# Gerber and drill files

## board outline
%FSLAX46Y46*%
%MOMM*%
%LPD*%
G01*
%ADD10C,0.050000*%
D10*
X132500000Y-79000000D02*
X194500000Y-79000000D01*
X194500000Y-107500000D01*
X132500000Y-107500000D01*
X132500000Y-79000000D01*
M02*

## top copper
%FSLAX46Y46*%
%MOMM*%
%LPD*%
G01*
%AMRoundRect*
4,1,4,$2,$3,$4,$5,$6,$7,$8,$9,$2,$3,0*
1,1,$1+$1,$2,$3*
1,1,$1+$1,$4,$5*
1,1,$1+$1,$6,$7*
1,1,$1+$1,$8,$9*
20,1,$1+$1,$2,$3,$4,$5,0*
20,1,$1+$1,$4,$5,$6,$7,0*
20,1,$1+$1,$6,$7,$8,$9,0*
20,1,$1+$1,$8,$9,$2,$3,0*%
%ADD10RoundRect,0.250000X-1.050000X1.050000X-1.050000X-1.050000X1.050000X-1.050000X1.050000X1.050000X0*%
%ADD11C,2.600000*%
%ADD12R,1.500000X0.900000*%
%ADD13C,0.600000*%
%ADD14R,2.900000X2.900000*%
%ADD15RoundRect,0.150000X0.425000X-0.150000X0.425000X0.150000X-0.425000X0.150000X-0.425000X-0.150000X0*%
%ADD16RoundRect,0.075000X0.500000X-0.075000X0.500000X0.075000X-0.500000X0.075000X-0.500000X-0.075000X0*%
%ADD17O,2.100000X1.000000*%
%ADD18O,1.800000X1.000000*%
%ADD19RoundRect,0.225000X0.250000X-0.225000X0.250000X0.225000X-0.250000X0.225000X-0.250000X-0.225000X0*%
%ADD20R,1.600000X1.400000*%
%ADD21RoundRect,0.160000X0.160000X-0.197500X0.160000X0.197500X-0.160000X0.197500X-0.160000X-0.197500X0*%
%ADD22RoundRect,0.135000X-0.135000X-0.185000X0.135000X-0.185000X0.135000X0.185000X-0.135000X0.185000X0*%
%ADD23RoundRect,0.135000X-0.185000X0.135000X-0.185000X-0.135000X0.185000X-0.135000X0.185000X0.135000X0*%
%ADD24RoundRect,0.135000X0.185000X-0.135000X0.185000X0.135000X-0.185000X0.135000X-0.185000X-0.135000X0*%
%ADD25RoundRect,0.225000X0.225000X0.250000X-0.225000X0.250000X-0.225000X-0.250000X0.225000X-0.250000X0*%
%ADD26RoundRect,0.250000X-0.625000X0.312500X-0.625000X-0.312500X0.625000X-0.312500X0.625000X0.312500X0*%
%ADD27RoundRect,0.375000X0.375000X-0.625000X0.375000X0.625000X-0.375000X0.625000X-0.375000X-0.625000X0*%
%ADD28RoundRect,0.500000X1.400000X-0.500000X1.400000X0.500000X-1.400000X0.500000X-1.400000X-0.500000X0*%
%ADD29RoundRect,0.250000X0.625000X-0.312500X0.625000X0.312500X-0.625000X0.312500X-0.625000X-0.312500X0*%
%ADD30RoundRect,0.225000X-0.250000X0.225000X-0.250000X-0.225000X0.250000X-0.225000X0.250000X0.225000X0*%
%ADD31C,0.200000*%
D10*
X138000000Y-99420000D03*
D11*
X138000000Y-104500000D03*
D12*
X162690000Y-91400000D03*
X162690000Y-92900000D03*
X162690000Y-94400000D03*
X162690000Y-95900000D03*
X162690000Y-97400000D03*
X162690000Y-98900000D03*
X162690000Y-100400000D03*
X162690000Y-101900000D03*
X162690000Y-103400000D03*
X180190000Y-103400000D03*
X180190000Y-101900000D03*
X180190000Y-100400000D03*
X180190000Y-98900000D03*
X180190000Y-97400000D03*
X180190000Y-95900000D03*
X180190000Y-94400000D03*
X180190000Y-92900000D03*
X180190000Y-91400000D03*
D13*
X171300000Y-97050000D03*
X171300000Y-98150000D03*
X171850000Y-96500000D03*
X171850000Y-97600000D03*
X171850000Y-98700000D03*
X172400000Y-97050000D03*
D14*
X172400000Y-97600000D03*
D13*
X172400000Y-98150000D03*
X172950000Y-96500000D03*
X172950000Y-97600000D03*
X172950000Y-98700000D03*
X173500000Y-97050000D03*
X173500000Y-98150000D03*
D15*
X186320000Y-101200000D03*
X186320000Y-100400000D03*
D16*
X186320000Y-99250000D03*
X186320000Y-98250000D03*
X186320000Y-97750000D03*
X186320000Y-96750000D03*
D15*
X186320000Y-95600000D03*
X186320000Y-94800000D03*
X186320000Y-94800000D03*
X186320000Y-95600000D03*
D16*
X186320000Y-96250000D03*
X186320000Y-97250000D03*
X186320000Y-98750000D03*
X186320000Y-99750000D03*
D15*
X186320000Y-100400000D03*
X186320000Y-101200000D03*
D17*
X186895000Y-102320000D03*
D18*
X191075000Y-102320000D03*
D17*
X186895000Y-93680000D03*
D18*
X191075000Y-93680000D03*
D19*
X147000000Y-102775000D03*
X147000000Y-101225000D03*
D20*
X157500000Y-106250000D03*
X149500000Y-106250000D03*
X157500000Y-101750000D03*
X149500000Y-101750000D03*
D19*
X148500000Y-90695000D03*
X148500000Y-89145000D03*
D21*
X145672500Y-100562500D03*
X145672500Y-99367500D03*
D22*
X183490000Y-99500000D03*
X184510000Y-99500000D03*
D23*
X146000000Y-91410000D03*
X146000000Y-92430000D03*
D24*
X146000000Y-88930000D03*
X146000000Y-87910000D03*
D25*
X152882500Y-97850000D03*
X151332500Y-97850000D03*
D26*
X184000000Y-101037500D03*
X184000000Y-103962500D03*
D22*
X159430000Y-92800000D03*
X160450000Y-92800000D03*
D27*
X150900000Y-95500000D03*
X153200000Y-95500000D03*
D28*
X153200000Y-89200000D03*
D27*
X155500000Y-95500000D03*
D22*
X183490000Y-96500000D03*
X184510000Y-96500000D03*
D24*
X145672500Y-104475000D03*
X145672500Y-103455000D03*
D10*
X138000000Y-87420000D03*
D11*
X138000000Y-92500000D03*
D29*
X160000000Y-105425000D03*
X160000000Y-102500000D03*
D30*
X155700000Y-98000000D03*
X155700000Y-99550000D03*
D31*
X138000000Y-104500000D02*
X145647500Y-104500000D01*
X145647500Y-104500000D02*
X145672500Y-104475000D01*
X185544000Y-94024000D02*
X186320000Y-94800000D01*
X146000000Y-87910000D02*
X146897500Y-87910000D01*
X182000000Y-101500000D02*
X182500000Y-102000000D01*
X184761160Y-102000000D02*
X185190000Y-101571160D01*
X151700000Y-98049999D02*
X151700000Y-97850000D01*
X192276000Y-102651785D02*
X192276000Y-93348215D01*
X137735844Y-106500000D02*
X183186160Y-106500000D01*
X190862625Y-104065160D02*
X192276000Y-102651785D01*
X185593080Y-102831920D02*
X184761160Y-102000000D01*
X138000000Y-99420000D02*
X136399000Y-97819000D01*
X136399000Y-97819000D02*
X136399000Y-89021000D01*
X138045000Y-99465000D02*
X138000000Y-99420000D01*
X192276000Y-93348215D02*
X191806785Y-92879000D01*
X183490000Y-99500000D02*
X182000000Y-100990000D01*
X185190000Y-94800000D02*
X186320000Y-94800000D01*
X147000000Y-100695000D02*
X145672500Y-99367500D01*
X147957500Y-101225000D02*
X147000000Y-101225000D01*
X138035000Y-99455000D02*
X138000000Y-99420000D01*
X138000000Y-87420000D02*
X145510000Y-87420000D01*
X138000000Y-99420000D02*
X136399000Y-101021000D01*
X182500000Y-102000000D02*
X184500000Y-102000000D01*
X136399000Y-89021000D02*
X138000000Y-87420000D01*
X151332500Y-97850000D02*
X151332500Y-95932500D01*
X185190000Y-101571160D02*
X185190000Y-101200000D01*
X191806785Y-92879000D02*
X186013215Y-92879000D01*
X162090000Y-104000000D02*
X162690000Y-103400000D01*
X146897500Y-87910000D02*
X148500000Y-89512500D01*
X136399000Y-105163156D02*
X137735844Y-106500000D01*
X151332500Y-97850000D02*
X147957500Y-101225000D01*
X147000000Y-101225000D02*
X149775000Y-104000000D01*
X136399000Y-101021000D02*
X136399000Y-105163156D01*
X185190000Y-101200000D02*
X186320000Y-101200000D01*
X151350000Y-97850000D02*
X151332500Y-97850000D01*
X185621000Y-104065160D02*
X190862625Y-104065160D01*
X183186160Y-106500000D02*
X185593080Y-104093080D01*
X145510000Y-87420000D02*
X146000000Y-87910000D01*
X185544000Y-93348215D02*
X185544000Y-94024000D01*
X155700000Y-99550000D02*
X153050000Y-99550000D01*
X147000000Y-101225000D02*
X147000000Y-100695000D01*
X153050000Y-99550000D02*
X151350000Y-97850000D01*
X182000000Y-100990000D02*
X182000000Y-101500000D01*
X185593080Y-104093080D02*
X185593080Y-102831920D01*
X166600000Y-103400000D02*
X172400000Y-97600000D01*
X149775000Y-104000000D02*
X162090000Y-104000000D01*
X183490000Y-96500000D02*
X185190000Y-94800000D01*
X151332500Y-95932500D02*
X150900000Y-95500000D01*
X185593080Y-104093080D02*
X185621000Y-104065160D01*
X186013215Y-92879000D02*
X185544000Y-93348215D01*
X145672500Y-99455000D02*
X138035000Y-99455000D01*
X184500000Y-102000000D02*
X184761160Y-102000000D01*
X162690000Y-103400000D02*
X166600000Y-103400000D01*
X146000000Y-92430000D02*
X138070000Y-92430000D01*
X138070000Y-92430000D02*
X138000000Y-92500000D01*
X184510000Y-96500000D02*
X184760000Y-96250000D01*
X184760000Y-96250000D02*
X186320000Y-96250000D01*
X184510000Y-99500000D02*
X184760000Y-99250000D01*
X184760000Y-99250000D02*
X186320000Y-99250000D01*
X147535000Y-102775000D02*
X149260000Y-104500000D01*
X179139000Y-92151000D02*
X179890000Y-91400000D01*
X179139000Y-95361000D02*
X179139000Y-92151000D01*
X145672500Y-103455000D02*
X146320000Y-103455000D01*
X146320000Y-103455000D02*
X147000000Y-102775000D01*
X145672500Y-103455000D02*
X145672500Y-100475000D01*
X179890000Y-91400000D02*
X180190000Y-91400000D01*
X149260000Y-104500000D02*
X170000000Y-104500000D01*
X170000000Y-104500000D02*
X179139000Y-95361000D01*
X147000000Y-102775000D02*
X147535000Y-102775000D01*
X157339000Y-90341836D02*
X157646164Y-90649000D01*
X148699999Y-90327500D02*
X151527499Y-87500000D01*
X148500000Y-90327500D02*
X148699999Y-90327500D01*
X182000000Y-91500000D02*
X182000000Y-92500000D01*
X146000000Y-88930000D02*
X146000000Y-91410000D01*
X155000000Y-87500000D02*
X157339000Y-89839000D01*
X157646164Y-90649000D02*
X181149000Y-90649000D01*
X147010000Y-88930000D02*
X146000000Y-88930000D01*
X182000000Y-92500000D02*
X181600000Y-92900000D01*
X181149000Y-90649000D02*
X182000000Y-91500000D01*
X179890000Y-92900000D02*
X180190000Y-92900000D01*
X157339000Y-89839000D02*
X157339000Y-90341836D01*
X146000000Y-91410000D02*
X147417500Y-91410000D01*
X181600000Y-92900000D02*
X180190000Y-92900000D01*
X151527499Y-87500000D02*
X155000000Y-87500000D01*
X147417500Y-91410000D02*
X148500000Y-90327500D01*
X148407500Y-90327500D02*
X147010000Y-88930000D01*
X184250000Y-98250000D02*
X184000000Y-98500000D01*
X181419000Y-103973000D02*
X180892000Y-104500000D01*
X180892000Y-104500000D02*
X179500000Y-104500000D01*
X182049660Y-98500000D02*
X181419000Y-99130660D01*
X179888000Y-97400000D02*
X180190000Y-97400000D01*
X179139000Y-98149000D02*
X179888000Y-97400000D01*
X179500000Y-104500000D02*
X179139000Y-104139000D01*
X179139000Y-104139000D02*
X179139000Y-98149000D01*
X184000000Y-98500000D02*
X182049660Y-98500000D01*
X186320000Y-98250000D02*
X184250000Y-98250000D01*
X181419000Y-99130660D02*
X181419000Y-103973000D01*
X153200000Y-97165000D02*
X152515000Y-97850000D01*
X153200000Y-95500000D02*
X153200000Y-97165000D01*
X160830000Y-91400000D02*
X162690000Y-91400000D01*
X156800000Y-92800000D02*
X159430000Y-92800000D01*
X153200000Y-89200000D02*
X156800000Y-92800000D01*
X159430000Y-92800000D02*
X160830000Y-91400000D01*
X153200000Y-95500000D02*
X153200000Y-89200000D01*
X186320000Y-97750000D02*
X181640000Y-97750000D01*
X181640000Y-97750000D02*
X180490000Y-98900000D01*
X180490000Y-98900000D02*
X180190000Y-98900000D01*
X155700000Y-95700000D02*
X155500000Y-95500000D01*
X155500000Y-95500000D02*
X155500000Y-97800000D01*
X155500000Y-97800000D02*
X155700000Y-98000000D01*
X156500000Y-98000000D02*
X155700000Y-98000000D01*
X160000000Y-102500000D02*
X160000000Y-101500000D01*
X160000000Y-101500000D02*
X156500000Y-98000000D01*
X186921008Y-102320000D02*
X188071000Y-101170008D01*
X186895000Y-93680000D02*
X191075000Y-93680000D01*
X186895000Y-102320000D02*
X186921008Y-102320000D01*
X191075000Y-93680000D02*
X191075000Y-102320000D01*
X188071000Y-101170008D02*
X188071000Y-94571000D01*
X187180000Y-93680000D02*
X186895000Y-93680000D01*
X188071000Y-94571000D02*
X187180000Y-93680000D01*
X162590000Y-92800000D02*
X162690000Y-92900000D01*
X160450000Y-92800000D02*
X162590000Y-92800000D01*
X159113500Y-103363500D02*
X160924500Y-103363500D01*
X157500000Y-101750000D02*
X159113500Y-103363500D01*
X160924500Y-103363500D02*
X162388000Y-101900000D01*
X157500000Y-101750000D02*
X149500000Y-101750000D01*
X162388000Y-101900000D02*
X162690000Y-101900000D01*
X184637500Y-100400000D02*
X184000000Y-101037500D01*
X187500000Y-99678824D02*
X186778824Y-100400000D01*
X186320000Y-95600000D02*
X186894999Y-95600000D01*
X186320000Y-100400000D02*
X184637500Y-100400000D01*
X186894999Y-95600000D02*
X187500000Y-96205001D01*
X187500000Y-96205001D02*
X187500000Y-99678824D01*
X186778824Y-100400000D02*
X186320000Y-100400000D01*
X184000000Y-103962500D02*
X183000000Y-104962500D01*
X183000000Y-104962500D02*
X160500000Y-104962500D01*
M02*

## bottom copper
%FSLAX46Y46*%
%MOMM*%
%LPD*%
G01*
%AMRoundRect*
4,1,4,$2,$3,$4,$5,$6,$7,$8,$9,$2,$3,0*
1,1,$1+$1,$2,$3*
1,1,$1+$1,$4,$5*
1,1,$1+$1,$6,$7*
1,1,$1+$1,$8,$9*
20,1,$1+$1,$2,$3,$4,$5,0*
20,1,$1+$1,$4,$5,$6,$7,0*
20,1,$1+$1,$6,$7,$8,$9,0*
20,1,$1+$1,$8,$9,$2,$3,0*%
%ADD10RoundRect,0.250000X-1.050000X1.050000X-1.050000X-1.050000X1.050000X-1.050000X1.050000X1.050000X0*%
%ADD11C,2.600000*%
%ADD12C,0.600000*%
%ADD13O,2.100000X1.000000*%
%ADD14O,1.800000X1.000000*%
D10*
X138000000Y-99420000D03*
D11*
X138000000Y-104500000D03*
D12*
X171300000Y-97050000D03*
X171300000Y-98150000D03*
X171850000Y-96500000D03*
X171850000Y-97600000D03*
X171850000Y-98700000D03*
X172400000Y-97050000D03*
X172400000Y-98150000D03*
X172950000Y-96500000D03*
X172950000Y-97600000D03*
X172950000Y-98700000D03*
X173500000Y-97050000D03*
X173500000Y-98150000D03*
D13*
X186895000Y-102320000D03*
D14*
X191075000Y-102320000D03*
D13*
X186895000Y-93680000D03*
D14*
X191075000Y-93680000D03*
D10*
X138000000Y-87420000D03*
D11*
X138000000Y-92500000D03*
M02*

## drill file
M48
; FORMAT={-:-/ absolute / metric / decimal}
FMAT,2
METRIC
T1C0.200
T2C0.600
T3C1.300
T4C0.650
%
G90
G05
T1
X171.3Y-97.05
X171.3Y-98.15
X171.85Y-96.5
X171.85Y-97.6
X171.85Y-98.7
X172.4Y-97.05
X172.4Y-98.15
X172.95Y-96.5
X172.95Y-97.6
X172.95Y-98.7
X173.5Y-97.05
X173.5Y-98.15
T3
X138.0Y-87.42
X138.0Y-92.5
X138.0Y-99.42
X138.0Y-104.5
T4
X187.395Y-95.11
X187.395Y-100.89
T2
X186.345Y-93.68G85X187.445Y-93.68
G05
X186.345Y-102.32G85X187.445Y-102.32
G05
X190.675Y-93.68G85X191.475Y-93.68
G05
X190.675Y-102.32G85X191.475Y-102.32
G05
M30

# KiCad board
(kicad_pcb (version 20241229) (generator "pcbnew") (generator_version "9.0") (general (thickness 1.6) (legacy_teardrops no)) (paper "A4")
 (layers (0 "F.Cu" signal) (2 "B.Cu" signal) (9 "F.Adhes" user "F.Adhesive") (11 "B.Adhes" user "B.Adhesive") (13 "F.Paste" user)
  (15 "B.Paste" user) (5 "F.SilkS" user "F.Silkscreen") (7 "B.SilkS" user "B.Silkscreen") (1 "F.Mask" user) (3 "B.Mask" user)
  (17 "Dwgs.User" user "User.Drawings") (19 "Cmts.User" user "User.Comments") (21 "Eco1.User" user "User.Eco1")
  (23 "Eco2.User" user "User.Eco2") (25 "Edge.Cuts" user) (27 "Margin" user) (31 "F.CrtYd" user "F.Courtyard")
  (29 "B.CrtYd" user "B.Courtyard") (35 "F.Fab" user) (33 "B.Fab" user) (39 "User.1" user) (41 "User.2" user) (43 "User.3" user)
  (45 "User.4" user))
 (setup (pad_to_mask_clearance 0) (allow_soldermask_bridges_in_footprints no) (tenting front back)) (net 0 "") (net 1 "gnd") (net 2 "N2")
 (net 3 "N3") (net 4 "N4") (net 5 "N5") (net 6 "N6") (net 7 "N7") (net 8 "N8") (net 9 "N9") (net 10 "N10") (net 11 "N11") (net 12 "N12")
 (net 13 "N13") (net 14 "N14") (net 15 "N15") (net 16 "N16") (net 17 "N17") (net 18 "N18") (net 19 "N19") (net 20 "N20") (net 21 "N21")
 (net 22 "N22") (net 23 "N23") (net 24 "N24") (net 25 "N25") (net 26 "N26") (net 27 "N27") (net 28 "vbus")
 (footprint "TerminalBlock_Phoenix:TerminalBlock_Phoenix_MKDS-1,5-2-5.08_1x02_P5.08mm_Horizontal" (layer "F.Cu") (at 138 99.42 -90)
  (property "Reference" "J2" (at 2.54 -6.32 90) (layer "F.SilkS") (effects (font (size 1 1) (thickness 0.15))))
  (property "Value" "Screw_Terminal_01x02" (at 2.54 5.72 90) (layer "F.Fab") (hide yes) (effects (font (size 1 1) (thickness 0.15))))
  (pad "1" thru_hole roundrect (at 0 0 270) (size 2.6 2.6) (drill 1.3) (layers "*.Cu" "*.Mask") (remove_unused_layers no)
   (roundrect_rratio 0.096154) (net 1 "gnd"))
  (pad "2" thru_hole circle (at 5.08 0 270) (size 2.6 2.6) (drill 1.3) (layers "*.Cu" "*.Mask") (remove_unused_layers no) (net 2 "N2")))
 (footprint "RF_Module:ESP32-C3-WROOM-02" (layer "F.Cu") (at 171.44 97.4)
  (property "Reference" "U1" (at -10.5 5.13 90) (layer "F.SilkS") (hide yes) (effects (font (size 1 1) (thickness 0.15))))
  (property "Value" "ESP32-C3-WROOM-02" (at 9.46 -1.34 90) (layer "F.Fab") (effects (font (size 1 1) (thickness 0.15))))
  (pad "" smd rect (at -0.14 -0.9) (size 0.7 0.7) (layers "F.Paste"))
  (pad "" smd rect (at -0.14 0.2) (size 0.7 0.7) (layers "F.Paste"))
  (pad "" smd rect (at -0.14 1.3) (size 0.7 0.7) (layers "F.Paste"))
  (pad "" smd rect (at 0.96 -0.9) (size 0.7 0.7) (layers "F.Paste"))
  (pad "" smd rect (at 0.96 0.2) (size 0.7 0.7) (layers "F.Paste"))
  (pad "" smd rect (at 0.96 1.3) (size 0.7 0.7) (layers "F.Paste"))
  (pad "" smd rect (at 2.06 -0.9) (size 0.7 0.7) (layers "F.Paste"))
  (pad "" smd rect (at 2.06 0.2) (size 0.7 0.7) (layers "F.Paste"))
  (pad "" smd rect (at 2.06 1.3) (size 0.7 0.7) (layers "F.Paste"))
  (pad "1" smd rect (at -8.75 -6) (size 1.5 0.9) (layers "F.Cu" "F.Mask" "F.Paste") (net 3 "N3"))
  (pad "2" smd rect (at -8.75 -4.5) (size 1.5 0.9) (layers "F.Cu" "F.Mask" "F.Paste") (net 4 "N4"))
  (pad "3" smd rect (at -8.75 -3) (size 1.5 0.9) (layers "F.Cu" "F.Mask" "F.Paste") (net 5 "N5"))
  (pad "4" smd rect (at -8.75 -1.5) (size 1.5 0.9) (layers "F.Cu" "F.Mask" "F.Paste") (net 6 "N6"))
  (pad "5" smd rect (at -8.75 0) (size 1.5 0.9) (layers "F.Cu" "F.Mask" "F.Paste") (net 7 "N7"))
  (pad "6" smd rect (at -8.75 1.5) (size 1.5 0.9) (layers "F.Cu" "F.Mask" "F.Paste") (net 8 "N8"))
  (pad "7" smd rect (at -8.75 3) (size 1.5 0.9) (layers "F.Cu" "F.Mask" "F.Paste") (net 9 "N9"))
  (pad "8" smd rect (at -8.75 4.5) (size 1.5 0.9) (layers "F.Cu" "F.Mask" "F.Paste") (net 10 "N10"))
  (pad "9" smd rect (at -8.75 6) (size 1.5 0.9) (layers "F.Cu" "F.Mask" "F.Paste") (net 1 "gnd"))
  (pad "10" smd rect (at 8.75 6) (size 1.5 0.9) (layers "F.Cu" "F.Mask" "F.Paste") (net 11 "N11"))
  (pad "11" smd rect (at 8.75 4.5) (size 1.5 0.9) (layers "F.Cu" "F.Mask" "F.Paste") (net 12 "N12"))
  (pad "12" smd rect (at 8.75 3) (size 1.5 0.9) (layers "F.Cu" "F.Mask" "F.Paste") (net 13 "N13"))
  (pad "13" smd rect (at 8.75 1.5) (size 1.5 0.9) (layers "F.Cu" "F.Mask" "F.Paste") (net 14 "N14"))
  (pad "14" smd rect (at 8.75 0) (size 1.5 0.9) (layers "F.Cu" "F.Mask" "F.Paste") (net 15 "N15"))
  (pad "15" smd rect (at 8.75 -1.5) (size 1.5 0.9) (layers "F.Cu" "F.Mask" "F.Paste") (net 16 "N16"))
  (pad "16" smd rect (at 8.75 -3) (size 1.5 0.9) (layers "F.Cu" "F.Mask" "F.Paste") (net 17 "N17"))
  (pad "17" smd rect (at 8.75 -4.5) (size 1.5 0.9) (layers "F.Cu" "F.Mask" "F.Paste") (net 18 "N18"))
  (pad "18" smd rect (at 8.75 -6) (size 1.5 0.9) (layers "F.Cu" "F.Mask" "F.Paste") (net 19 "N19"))
  (pad "19" thru_hole circle (at -0.14 -0.35) (size 0.6 0.6) (drill 0.2) (layers "*.Cu" "F.Mask") (remove_unused_layers no) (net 1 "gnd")
   (zone_connect 2))
  (pad "19" thru_hole circle (at -0.14 0.75) (size 0.6 0.6) (drill 0.2) (layers "*.Cu" "F.Mask") (remove_unused_layers no) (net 1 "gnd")
   (zone_connect 2))
  (pad "19" thru_hole circle (at 0.41 -0.9) (size 0.6 0.6) (drill 0.2) (layers "*.Cu" "F.Mask") (remove_unused_layers no) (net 1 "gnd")
   (zone_connect 2))
  (pad "19" thru_hole circle (at 0.41 0.2) (size 0.6 0.6) (drill 0.2) (layers "*.Cu" "F.Mask") (remove_unused_layers no) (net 1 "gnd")
   (zone_connect 2))
  (pad "19" thru_hole circle (at 0.41 1.3) (size 0.6 0.6) (drill 0.2) (layers "*.Cu" "F.Mask") (remove_unused_layers no) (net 1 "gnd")
   (zone_connect 2))
  (pad "19" thru_hole circle (at 0.96 -0.35) (size 0.6 0.6) (drill 0.2) (layers "*.Cu" "F.Mask") (remove_unused_layers no) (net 1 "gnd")
   (zone_connect 2))
  (pad "19" smd rect (at 0.96 0.2) (size 2.9 2.9) (layers "F.Cu" "F.Mask") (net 1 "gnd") (zone_connect 2))
  (pad "19" thru_hole circle (at 0.96 0.75) (size 0.6 0.6) (drill 0.2) (layers "*.Cu" "F.Mask") (remove_unused_layers no) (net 1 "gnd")
   (zone_connect 2))
  (pad "19" thru_hole circle (at 1.51 -0.9) (size 0.6 0.6) (drill 0.2) (layers "*.Cu" "F.Mask") (remove_unused_layers no) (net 1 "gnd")
   (zone_connect 2))
  (pad "19" thru_hole circle (at 1.51 0.2) (size 0.6 0.6) (drill 0.2) (layers "*.Cu" "F.Mask") (remove_unused_layers no) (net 1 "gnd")
   (zone_connect 2))
  (pad "19" thru_hole circle (at 1.51 1.3) (size 0.6 0.6) (drill 0.2) (layers "*.Cu" "F.Mask") (remove_unused_layers no) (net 1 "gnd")
   (zone_connect 2))
  (pad "19" thru_hole circle (at 2.06 -0.35) (size 0.6 0.6) (drill 0.2) (layers "*.Cu" "F.Mask") (remove_unused_layers no) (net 1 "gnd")
   (zone_connect 2))
  (pad "19" thru_hole circle (at 2.06 0.75) (size 0.6 0.6) (drill 0.2) (layers "*.Cu" "F.Mask") (remove_unused_layers no) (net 1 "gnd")
   (zone_connect 2))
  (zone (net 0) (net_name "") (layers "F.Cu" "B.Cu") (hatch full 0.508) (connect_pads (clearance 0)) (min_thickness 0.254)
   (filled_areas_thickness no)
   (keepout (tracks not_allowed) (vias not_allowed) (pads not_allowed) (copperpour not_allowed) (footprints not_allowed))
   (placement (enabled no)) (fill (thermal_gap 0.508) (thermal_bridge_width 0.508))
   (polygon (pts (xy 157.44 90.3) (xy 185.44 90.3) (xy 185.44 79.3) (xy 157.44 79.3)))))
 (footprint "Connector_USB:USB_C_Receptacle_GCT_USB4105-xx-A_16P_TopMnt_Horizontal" (layer "F.Cu") (at 190 98 90)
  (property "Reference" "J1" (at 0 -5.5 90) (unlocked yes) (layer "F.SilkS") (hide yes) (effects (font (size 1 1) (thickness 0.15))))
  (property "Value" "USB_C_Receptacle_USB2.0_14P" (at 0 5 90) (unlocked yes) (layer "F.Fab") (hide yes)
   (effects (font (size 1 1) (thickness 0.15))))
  (pad "" np_thru_hole circle (at -2.89 -2.605 90) (size 0.65 0.65) (drill 0.65) (layers "*.Cu" "*.Mask"))
  (pad "" np_thru_hole circle (at 2.89 -2.605 90) (size 0.65 0.65) (drill 0.65) (layers "*.Cu" "*.Mask"))
  (pad "A1" smd roundrect (at -3.2 -3.68 90) (size 0.6 1.15) (layers "F.Cu" "F.Mask" "F.Paste") (roundrect_rratio 0.25) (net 1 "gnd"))
  (pad "A4" smd roundrect (at -2.4 -3.68 90) (size 0.6 1.15) (layers "F.Cu" "F.Mask" "F.Paste") (roundrect_rratio 0.25) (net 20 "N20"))
  (pad "A5" smd roundrect (at -1.25 -3.68 90) (size 0.3 1.15) (layers "F.Cu" "F.Mask" "F.Paste") (roundrect_rratio 0.25) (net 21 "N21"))
  (pad "A6" smd roundrect (at -0.25 -3.68 90) (size 0.3 1.15) (layers "F.Cu" "F.Mask" "F.Paste") (roundrect_rratio 0.25) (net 15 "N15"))
  (pad "A7" smd roundrect (at 0.25 -3.68 90) (size 0.3 1.15) (layers "F.Cu" "F.Mask" "F.Paste") (roundrect_rratio 0.25) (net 14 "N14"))
  (pad "A8" smd roundrect (at 1.25 -3.68 90) (size 0.3 1.15) (layers "F.Cu" "F.Mask" "F.Paste") (roundrect_rratio 0.25))
  (pad "A9" smd roundrect (at 2.4 -3.68 90) (size 0.6 1.15) (layers "F.Cu" "F.Mask" "F.Paste") (roundrect_rratio 0.25) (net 20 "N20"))
  (pad "A12" smd roundrect (at 3.2 -3.68 90) (size 0.6 1.15) (layers "F.Cu" "F.Mask" "F.Paste") (roundrect_rratio 0.25) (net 1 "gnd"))
  (pad "B1" smd roundrect (at 3.2 -3.68 90) (size 0.6 1.15) (layers "F.Cu" "F.Mask" "F.Paste") (roundrect_rratio 0.25) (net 1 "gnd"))
  (pad "B4" smd roundrect (at 2.4 -3.68 90) (size 0.6 1.15) (layers "F.Cu" "F.Mask" "F.Paste") (roundrect_rratio 0.25) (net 20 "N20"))
  (pad "B5" smd roundrect (at 1.75 -3.68 90) (size 0.3 1.15) (layers "F.Cu" "F.Mask" "F.Paste") (roundrect_rratio 0.25) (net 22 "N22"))
  (pad "B6" smd roundrect (at 0.75 -3.68 90) (size 0.3 1.15) (layers "F.Cu" "F.Mask" "F.Paste") (roundrect_rratio 0.25) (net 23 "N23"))
  (pad "B7" smd roundrect (at -0.75 -3.68 90) (size 0.3 1.15) (layers "F.Cu" "F.Mask" "F.Paste") (roundrect_rratio 0.25) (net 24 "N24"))
  (pad "B8" smd roundrect (at -1.75 -3.68 90) (size 0.3 1.15) (layers "F.Cu" "F.Mask" "F.Paste") (roundrect_rratio 0.25))
  (pad "B9" smd roundrect (at -2.4 -3.68 90) (size 0.6 1.15) (layers "F.Cu" "F.Mask" "F.Paste") (roundrect_rratio 0.25) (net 20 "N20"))
  (pad "B12" smd roundrect (at -3.2 -3.68 90) (size 0.6 1.15) (layers "F.Cu" "F.Mask" "F.Paste") (roundrect_rratio 0.25) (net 1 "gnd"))
  (pad "S1" thru_hole oval (at -4.32 -3.105 90) (size 1 2.1) (drill oval 0.6 1.7) (layers "*.Cu" "*.Mask" "F.Paste")
   (remove_unused_layers no) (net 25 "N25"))
  (pad "S1" thru_hole oval (at -4.32 1.075 90) (size 1 1.8) (drill oval 0.6 1.4) (layers "*.Cu" "*.Mask" "F.Paste")
   (remove_unused_layers no) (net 25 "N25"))
  (pad "S1" thru_hole oval (at 4.32 -3.105 90) (size 1 2.1) (drill oval 0.6 1.7) (layers "*.Cu" "*.Mask" "F.Paste")
   (remove_unused_layers no) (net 25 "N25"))
  (pad "S1" thru_hole oval (at 4.32 1.075 90) (size 1 1.8) (drill oval 0.6 1.4) (layers "*.Cu" "*.Mask" "F.Paste") (remove_unused_layers no)
   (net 25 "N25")))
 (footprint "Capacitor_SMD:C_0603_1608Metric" (layer "F.Cu") (at 147 102 90)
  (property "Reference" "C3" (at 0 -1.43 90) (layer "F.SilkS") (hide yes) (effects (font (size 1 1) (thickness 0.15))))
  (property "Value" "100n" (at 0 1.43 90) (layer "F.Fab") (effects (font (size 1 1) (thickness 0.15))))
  (pad "1" smd roundrect (at -0.775 0 90) (size 0.9 0.95) (layers "F.Cu" "F.Mask" "F.Paste") (roundrect_rratio 0.25) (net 19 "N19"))
  (pad "2" smd roundrect (at 0.775 0 90) (size 0.9 0.95) (layers "F.Cu" "F.Mask" "F.Paste") (roundrect_rratio 0.25) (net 1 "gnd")))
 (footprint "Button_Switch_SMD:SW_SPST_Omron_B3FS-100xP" (layer "F.Cu") (at 153.5 104 180)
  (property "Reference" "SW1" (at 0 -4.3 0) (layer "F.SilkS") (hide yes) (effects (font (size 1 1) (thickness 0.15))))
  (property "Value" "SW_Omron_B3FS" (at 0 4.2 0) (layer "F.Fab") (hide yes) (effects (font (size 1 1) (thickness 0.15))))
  (pad "1" smd rect (at -4 -2.25) (size 1.6 1.4) (layers "F.Cu" "F.Mask" "F.Paste") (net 1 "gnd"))
  (pad "1" smd rect (at 4 -2.25) (size 1.6 1.4) (layers "F.Cu" "F.Mask" "F.Paste") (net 1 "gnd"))
  (pad "2" smd rect (at -4 2.25) (size 1.6 1.4) (layers "F.Cu" "F.Mask" "F.Paste") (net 10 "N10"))
  (pad "2" smd rect (at 4 2.25) (size 1.6 1.4) (layers "F.Cu" "F.Mask" "F.Paste") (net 10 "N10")))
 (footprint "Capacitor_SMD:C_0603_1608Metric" (layer "F.Cu") (at 148.5 89.92 90)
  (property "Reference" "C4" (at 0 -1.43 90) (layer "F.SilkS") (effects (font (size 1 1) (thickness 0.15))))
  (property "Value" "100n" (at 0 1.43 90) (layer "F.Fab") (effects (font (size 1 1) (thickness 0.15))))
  (pad "1" smd roundrect (at -0.775 0 90) (size 0.9 0.95) (layers "F.Cu" "F.Mask" "F.Paste") (roundrect_rratio 0.25) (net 18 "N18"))
  (pad "2" smd roundrect (at 0.775 0 90) (size 0.9 0.95) (layers "F.Cu" "F.Mask" "F.Paste") (roundrect_rratio 0.25) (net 1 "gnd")))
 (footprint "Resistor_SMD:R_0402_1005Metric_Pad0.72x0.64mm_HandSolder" (layer "F.Cu") (at 145.6725 99.965 90)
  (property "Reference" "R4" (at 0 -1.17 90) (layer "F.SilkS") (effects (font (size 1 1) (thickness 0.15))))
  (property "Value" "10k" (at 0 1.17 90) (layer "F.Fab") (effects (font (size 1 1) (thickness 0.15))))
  (pad "1" smd roundrect (at -0.5975 0 90) (size 0.715 0.64) (layers "F.Cu" "F.Mask" "F.Paste") (roundrect_rratio 0.25) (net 19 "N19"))
  (pad "2" smd roundrect (at 0.5975 0 90) (size 0.715 0.64) (layers "F.Cu" "F.Mask" "F.Paste") (roundrect_rratio 0.25) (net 1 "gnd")))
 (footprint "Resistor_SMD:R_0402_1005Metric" (layer "F.Cu") (at 184 99.5)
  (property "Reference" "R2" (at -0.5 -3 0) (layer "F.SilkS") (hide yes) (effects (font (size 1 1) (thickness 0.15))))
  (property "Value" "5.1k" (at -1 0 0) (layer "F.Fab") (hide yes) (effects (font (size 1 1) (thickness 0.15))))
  (pad "1" smd roundrect (at -0.51 0) (size 0.54 0.64) (layers "F.Cu" "F.Mask" "F.Paste") (roundrect_rratio 0.25) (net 1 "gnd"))
  (pad "2" smd roundrect (at 0.51 0) (size 0.54 0.64) (layers "F.Cu" "F.Mask" "F.Paste") (roundrect_rratio 0.25) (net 21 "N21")))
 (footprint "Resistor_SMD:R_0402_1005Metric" (layer "F.Cu") (at 146 91.92 -90)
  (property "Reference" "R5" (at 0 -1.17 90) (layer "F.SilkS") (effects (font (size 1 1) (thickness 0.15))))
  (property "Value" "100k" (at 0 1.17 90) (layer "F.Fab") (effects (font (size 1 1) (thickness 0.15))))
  (pad "1" smd roundrect (at -0.51 0 270) (size 0.54 0.64) (layers "F.Cu" "F.Mask" "F.Paste") (roundrect_rratio 0.25) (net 18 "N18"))
  (pad "2" smd roundrect (at 0.51 0 270) (size 0.54 0.64) (layers "F.Cu" "F.Mask" "F.Paste") (roundrect_rratio 0.25) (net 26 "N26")))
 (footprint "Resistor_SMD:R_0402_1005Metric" (layer "F.Cu") (at 146 88.42 90)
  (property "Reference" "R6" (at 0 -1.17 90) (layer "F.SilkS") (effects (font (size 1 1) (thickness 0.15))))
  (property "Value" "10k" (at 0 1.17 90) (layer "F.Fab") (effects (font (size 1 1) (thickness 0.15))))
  (pad "1" smd roundrect (at -0.51 0 90) (size 0.54 0.64) (layers "F.Cu" "F.Mask" "F.Paste") (roundrect_rratio 0.25) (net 18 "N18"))
  (pad "2" smd roundrect (at 0.51 0 90) (size 0.54 0.64) (layers "F.Cu" "F.Mask" "F.Paste") (roundrect_rratio 0.25) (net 1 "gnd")))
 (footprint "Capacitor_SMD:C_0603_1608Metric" (layer "F.Cu") (at 152.1075 97.85 180)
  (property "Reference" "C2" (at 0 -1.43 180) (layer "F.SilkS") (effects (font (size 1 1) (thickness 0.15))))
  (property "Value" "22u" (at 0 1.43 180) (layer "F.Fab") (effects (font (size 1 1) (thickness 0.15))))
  (pad "1" smd roundrect (at -0.775 0 180) (size 0.9 0.95) (layers "F.Cu" "F.Mask" "F.Paste") (roundrect_rratio 0.25) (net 3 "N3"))
  (pad "2" smd roundrect (at 0.775 0 180) (size 0.9 0.95) (layers "F.Cu" "F.Mask" "F.Paste") (roundrect_rratio 0.25) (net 1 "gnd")))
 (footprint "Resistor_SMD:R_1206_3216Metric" (layer "F.Cu") (at 184 102.5 -90)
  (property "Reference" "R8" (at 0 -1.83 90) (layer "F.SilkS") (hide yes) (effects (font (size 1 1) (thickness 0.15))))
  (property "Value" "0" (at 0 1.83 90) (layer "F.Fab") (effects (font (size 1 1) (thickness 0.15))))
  (pad "1" smd roundrect (at -1.4625 0 270) (size 1.125 1.75) (layers "F.Cu" "F.Mask" "F.Paste") (roundrect_rratio 0.222222) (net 20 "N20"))
  (pad "2" smd roundrect (at 1.4625 0 270) (size 1.125 1.75) (layers "F.Cu" "F.Mask" "F.Paste") (roundrect_rratio 0.222222) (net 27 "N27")))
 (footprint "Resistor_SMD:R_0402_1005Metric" (layer "F.Cu") (at 159.94 92.8)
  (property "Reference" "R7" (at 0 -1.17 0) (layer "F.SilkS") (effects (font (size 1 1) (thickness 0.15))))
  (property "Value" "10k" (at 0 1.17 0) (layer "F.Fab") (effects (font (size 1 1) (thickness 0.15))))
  (pad "1" smd roundrect (at -0.51 0) (size 0.54 0.64) (layers "F.Cu" "F.Mask" "F.Paste") (roundrect_rratio 0.25) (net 3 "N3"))
  (pad "2" smd roundrect (at 0.51 0) (size 0.54 0.64) (layers "F.Cu" "F.Mask" "F.Paste") (roundrect_rratio 0.25) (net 4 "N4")))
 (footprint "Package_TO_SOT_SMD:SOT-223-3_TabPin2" (layer "F.Cu") (at 153.2 92.35 90)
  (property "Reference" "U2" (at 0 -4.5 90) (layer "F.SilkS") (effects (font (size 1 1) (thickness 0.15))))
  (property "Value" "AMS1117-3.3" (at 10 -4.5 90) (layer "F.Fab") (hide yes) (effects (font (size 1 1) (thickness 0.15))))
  (pad "1" smd roundrect (at -3.15 -2.3 90) (size 2 1.5) (layers "F.Cu" "F.Mask" "F.Paste") (roundrect_rratio 0.25) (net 1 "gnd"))
  (pad "2" smd roundrect (at -3.15 0 90) (size 2 1.5) (layers "F.Cu" "F.Mask" "F.Paste") (roundrect_rratio 0.25) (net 3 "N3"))
  (pad "2" smd roundrect (at 3.15 0 90) (size 2 3.8) (layers "F.Cu" "F.Mask" "F.Paste") (roundrect_rratio 0.25) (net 3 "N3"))
  (pad "3" smd roundrect (at -3.15 2.3 90) (size 2 1.5) (layers "F.Cu" "F.Mask" "F.Paste") (roundrect_rratio 0.25) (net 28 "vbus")))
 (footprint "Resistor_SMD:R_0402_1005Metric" (layer "F.Cu") (at 184 96.5)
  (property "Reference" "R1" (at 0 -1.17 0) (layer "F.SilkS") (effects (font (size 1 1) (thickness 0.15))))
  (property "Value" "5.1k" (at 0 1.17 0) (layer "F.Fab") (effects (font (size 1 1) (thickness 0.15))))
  (pad "1" smd roundrect (at -0.51 0) (size 0.54 0.64) (layers "F.Cu" "F.Mask" "F.Paste") (roundrect_rratio 0.25) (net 1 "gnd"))
  (pad "2" smd roundrect (at 0.51 0) (size 0.54 0.64) (layers "F.Cu" "F.Mask" "F.Paste") (roundrect_rratio 0.25) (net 22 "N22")))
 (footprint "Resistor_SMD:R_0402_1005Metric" (layer "F.Cu") (at 145.6725 103.965 90)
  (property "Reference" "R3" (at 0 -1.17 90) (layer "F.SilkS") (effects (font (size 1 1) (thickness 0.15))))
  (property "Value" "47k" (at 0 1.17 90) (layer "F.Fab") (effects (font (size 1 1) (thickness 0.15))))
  (pad "1" smd roundrect (at -0.51 0 90) (size 0.54 0.64) (layers "F.Cu" "F.Mask" "F.Paste") (roundrect_rratio 0.25) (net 2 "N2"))
  (pad "2" smd roundrect (at 0.51 0 90) (size 0.54 0.64) (layers "F.Cu" "F.Mask" "F.Paste") (roundrect_rratio 0.25) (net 19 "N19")))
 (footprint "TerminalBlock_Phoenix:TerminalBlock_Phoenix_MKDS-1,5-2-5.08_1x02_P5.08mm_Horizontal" (layer "F.Cu") (at 138 87.42 -90)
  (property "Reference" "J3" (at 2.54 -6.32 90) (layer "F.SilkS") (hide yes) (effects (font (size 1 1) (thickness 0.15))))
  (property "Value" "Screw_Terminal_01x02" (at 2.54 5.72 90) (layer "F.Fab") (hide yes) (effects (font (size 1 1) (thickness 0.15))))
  (pad "1" thru_hole roundrect (at 0 0 270) (size 2.6 2.6) (drill 1.3) (layers "*.Cu" "*.Mask") (remove_unused_layers no)
   (roundrect_rratio 0.096154) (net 1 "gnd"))
  (pad "2" thru_hole circle (at 5.08 0 270) (size 2.6 2.6) (drill 1.3) (layers "*.Cu" "*.Mask") (remove_unused_layers no) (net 26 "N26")))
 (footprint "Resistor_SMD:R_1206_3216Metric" (layer "F.Cu") (at 160 103.9625 90)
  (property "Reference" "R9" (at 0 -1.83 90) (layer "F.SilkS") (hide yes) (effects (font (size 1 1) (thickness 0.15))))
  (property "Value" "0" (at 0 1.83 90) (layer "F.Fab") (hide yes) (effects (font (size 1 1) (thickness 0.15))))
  (pad "1" smd roundrect (at -1.4625 0 90) (size 1.125 1.75) (layers "F.Cu" "F.Mask" "F.Paste") (roundrect_rratio 0.222222) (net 27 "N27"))
  (pad "2" smd roundrect (at 1.4625 0 90) (size 1.125 1.75) (layers "F.Cu" "F.Mask" "F.Paste") (roundrect_rratio 0.222222) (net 28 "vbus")))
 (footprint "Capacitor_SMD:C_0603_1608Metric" (layer "F.Cu") (at 155.7 98.775 -90)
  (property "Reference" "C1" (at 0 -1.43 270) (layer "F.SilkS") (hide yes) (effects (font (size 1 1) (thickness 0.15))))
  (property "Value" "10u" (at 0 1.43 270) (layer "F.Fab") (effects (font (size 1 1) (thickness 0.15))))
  (pad "1" smd roundrect (at -0.775 0 270) (size 0.9 0.95) (layers "F.Cu" "F.Mask" "F.Paste") (roundrect_rratio 0.25) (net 28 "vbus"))
  (pad "2" smd roundrect (at 0.775 0 270) (size 0.9 0.95) (layers "F.Cu" "F.Mask" "F.Paste") (roundrect_rratio 0.25) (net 1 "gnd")))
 (gr_rect (start 132.5 79) (end 194.5 107.5) (stroke (width 0.05) (type default)) (fill no) (layer "Edge.Cuts"))
 (segment (start 138 104.5) (end 145.6475 104.5) (width 0.2) (layer "F.Cu") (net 2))
 (segment (start 145.6475 104.5) (end 145.6725 104.475) (width 0.2) (layer "F.Cu") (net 2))
 (segment (start 185.544 94.024) (end 186.32 94.8) (width 0.2) (layer "F.Cu") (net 1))
 (segment (start 146 87.91) (end 146.8975 87.91) (width 0.2) (layer "F.Cu") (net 1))
 (segment (start 182 101.5) (end 182.5 102) (width 0.2) (layer "F.Cu") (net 1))
 (segment (start 184.76116 102) (end 185.19 101.57116) (width 0.2) (layer "F.Cu") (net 1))
 (segment (start 151.7 98.049999) (end 151.7 97.85) (width 0.2) (layer "F.Cu") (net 1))
 (segment (start 192.276 102.651785) (end 192.276 93.348215) (width 0.2) (layer "F.Cu") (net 1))
 (segment (start 137.735844 106.5) (end 183.18616 106.5) (width 0.2) (layer "F.Cu") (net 1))
 (segment (start 190.862625 104.06516) (end 192.276 102.651785) (width 0.2) (layer "F.Cu") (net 1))
 (segment (start 185.59308 102.83192) (end 184.76116 102) (width 0.2) (layer "F.Cu") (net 1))
 (segment (start 138 99.42) (end 136.399 97.819) (width 0.2) (layer "F.Cu") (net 1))
 (segment (start 136.399 97.819) (end 136.399 89.021) (width 0.2) (layer "F.Cu") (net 1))
 (segment (start 138.045 99.465) (end 138 99.42) (width 0.2) (layer "F.Cu") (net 1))
 (segment (start 192.276 93.348215) (end 191.806785 92.879) (width 0.2) (layer "F.Cu") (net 1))
 (segment (start 183.49 99.5) (end 182 100.99) (width 0.2) (layer "F.Cu") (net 1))
 (segment (start 185.19 94.8) (end 186.32 94.8) (width 0.2) (layer "F.Cu") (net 1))
 (segment (start 147 100.695) (end 145.6725 99.3675) (width 0.2) (layer "F.Cu") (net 1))
 (segment (start 147.9575 101.225) (end 147 101.225) (width 0.2) (layer "F.Cu") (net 1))
 (segment (start 138.035 99.455) (end 138 99.42) (width 0.2) (layer "F.Cu") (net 1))
 (segment (start 138 87.42) (end 145.51 87.42) (width 0.2) (layer "F.Cu") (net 1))
 (segment (start 138 99.42) (end 136.399 101.021) (width 0.2) (layer "F.Cu") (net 1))
 (segment (start 182.5 102) (end 184.5 102) (width 0.2) (layer "F.Cu") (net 1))
 (segment (start 136.399 89.021) (end 138 87.42) (width 0.2) (layer "F.Cu") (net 1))
 (segment (start 151.3325 97.85) (end 151.3325 95.9325) (width 0.2) (layer "F.Cu") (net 1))
 (segment (start 185.19 101.57116) (end 185.19 101.2) (width 0.2) (layer "F.Cu") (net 1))
 (segment (start 191.806785 92.879) (end 186.013215 92.879) (width 0.2) (layer "F.Cu") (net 1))
 (segment (start 162.09 104) (end 162.69 103.4) (width 0.2) (layer "F.Cu") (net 1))
 (segment (start 146.8975 87.91) (end 148.5 89.5125) (width 0.2) (layer "F.Cu") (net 1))
 (segment (start 136.399 105.163156) (end 137.735844 106.5) (width 0.2) (layer "F.Cu") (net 1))
 (segment (start 151.3325 97.85) (end 147.9575 101.225) (width 0.2) (layer "F.Cu") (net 1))
 (segment (start 147 101.225) (end 149.775 104) (width 0.2) (layer "F.Cu") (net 1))
 (segment (start 136.399 101.021) (end 136.399 105.163156) (width 0.2) (layer "F.Cu") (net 1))
 (segment (start 185.19 101.2) (end 186.32 101.2) (width 0.2) (layer "F.Cu") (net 1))
 (segment (start 151.35 97.85) (end 151.3325 97.85) (width 0.2) (layer "F.Cu") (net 1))
 (segment (start 185.621 104.06516) (end 190.862625 104.06516) (width 0.2) (layer "F.Cu") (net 1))
 (segment (start 183.18616 106.5) (end 185.59308 104.09308) (width 0.2) (layer "F.Cu") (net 1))
 (segment (start 145.51 87.42) (end 146 87.91) (width 0.2) (layer "F.Cu") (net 1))
 (segment (start 185.544 93.348215) (end 185.544 94.024) (width 0.2) (layer "F.Cu") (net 1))
 (segment (start 155.7 99.55) (end 153.05 99.55) (width 0.2) (layer "F.Cu") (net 1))
 (segment (start 147 101.225) (end 147 100.695) (width 0.2) (layer "F.Cu") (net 1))
 (segment (start 153.05 99.55) (end 151.35 97.85) (width 0.2) (layer "F.Cu") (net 1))
 (segment (start 182 100.99) (end 182 101.5) (width 0.2) (layer "F.Cu") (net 1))
 (segment (start 185.59308 104.09308) (end 185.59308 102.83192) (width 0.2) (layer "F.Cu") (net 1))
 (segment (start 166.6 103.4) (end 172.4 97.6) (width 0.2) (layer "F.Cu") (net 1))
 (segment (start 149.775 104) (end 162.09 104) (width 0.2) (layer "F.Cu") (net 1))
 (segment (start 183.49 96.5) (end 185.19 94.8) (width 0.2) (layer "F.Cu") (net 1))
 (segment (start 151.3325 95.9325) (end 150.9 95.5) (width 0.2) (layer "F.Cu") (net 1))
 (segment (start 185.59308 104.09308) (end 185.621 104.06516) (width 0.2) (layer "F.Cu") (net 1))
 (segment (start 186.013215 92.879) (end 185.544 93.348215) (width 0.2) (layer "F.Cu") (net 1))
 (segment (start 145.6725 99.455) (end 138.035 99.455) (width 0.2) (layer "F.Cu") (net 1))
 (segment (start 184.5 102) (end 184.76116 102) (width 0.2) (layer "F.Cu") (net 1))
 (segment (start 162.69 103.4) (end 166.6 103.4) (width 0.2) (layer "F.Cu") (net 1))
 (segment (start 146 92.43) (end 138.07 92.43) (width 0.2) (layer "F.Cu") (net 26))
 (segment (start 138.07 92.43) (end 138 92.5) (width 0.2) (layer "F.Cu") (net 26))
 (segment (start 184.51 96.5) (end 184.76 96.25) (width 0.2) (layer "F.Cu") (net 22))
 (segment (start 184.76 96.25) (end 186.32 96.25) (width 0.2) (layer "F.Cu") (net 22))
 (segment (start 184.51 99.5) (end 184.76 99.25) (width 0.2) (layer "F.Cu") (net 21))
 (segment (start 184.76 99.25) (end 186.32 99.25) (width 0.2) (layer "F.Cu") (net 21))
 (segment (start 147.535 102.775) (end 149.26 104.5) (width 0.2) (layer "F.Cu") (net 19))
 (segment (start 179.139 92.151) (end 179.89 91.4) (width 0.2) (layer "F.Cu") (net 19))
 (segment (start 179.139 95.361) (end 179.139 92.151) (width 0.2) (layer "F.Cu") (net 19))
 (segment (start 145.6725 103.455) (end 146.32 103.455) (width 0.2) (layer "F.Cu") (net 19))
 (segment (start 146.32 103.455) (end 147 102.775) (width 0.2) (layer "F.Cu") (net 19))
 (segment (start 145.6725 103.455) (end 145.6725 100.475) (width 0.2) (layer "F.Cu") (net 19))
 (segment (start 179.89 91.4) (end 180.19 91.4) (width 0.2) (layer "F.Cu") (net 19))
 (segment (start 149.26 104.5) (end 170 104.5) (width 0.2) (layer "F.Cu") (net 19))
 (segment (start 170 104.5) (end 179.139 95.361) (width 0.2) (layer "F.Cu") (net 19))
 (segment (start 147 102.775) (end 147.535 102.775) (width 0.2) (layer "F.Cu") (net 19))
 (segment (start 157.339 90.341836) (end 157.646164 90.649) (width 0.2) (layer "F.Cu") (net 18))
 (segment (start 148.699999 90.3275) (end 151.527499 87.5) (width 0.2) (layer "F.Cu") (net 18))
 (segment (start 148.5 90.3275) (end 148.699999 90.3275) (width 0.2) (layer "F.Cu") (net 18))
 (segment (start 182 91.5) (end 182 92.5) (width 0.2) (layer "F.Cu") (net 18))
 (segment (start 146 88.93) (end 146 91.41) (width 0.2) (layer "F.Cu") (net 18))
 (segment (start 155 87.5) (end 157.339 89.839) (width 0.2) (layer "F.Cu") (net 18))
 (segment (start 157.646164 90.649) (end 181.149 90.649) (width 0.2) (layer "F.Cu") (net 18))
 (segment (start 147.01 88.93) (end 146 88.93) (width 0.2) (layer "F.Cu") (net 18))
 (segment (start 182 92.5) (end 181.6 92.9) (width 0.2) (layer "F.Cu") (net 18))
 (segment (start 181.149 90.649) (end 182 91.5) (width 0.2) (layer "F.Cu") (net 18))
 (segment (start 179.89 92.9) (end 180.19 92.9) (width 0.2) (layer "F.Cu") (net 18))
 (segment (start 157.339 89.839) (end 157.339 90.341836) (width 0.2) (layer "F.Cu") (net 18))
 (segment (start 146 91.41) (end 147.4175 91.41) (width 0.2) (layer "F.Cu") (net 18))
 (segment (start 181.6 92.9) (end 180.19 92.9) (width 0.2) (layer "F.Cu") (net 18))
 (segment (start 151.527499 87.5) (end 155 87.5) (width 0.2) (layer "F.Cu") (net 18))
 (segment (start 147.4175 91.41) (end 148.5 90.3275) (width 0.2) (layer "F.Cu") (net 18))
 (segment (start 148.4075 90.3275) (end 147.01 88.93) (width 0.2) (layer "F.Cu") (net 18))
 (segment (start 184.25 98.25) (end 184 98.5) (width 0.2) (layer "F.Cu") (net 15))
 (segment (start 181.419 103.973) (end 180.892 104.5) (width 0.2) (layer "F.Cu") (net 15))
 (segment (start 180.892 104.5) (end 179.5 104.5) (width 0.2) (layer "F.Cu") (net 15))
 (segment (start 182.04966 98.5) (end 181.419 99.13066) (width 0.2) (layer "F.Cu") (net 15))
 (segment (start 179.888 97.4) (end 180.19 97.4) (width 0.2) (layer "F.Cu") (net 15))
 (segment (start 179.139 98.149) (end 179.888 97.4) (width 0.2) (layer "F.Cu") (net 15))
 (segment (start 179.5 104.5) (end 179.139 104.139) (width 0.2) (layer "F.Cu") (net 15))
 (segment (start 179.139 104.139) (end 179.139 98.149) (width 0.2) (layer "F.Cu") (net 15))
 (segment (start 184 98.5) (end 182.04966 98.5) (width 0.2) (layer "F.Cu") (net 15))
 (segment (start 186.32 98.25) (end 184.25 98.25) (width 0.2) (layer "F.Cu") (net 15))
 (segment (start 181.419 99.13066) (end 181.419 103.973) (width 0.2) (layer "F.Cu") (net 15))
 (segment (start 153.2 97.165) (end 152.515 97.85) (width 0.2) (layer "F.Cu") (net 3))
 (segment (start 153.2 95.5) (end 153.2 97.165) (width 0.2) (layer "F.Cu") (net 3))
 (segment (start 160.83 91.4) (end 162.69 91.4) (width 0.2) (layer "F.Cu") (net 3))
 (segment (start 156.8 92.8) (end 159.43 92.8) (width 0.2) (layer "F.Cu") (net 3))
 (segment (start 153.2 89.2) (end 156.8 92.8) (width 0.2) (layer "F.Cu") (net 3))
 (segment (start 159.43 92.8) (end 160.83 91.4) (width 0.2) (layer "F.Cu") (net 3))
 (segment (start 153.2 95.5) (end 153.2 89.2) (width 0.2) (layer "F.Cu") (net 3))
 (segment (start 186.32 97.75) (end 181.64 97.75) (width 0.2) (layer "F.Cu") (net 14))
 (segment (start 181.64 97.75) (end 180.49 98.9) (width 0.2) (layer "F.Cu") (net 14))
 (segment (start 180.49 98.9) (end 180.19 98.9) (width 0.2) (layer "F.Cu") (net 14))
 (segment (start 155.7 95.7) (end 155.5 95.5) (width 0.2) (layer "F.Cu") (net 28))
 (segment (start 155.5 95.5) (end 155.5 97.8) (width 0.2) (layer "F.Cu") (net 28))
 (segment (start 155.5 97.8) (end 155.7 98) (width 0.2) (layer "F.Cu") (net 28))
 (segment (start 156.5 98) (end 155.7 98) (width 0.2) (layer "F.Cu") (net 28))
 (segment (start 160 102.5) (end 160 101.5) (width 0.2) (layer "F.Cu") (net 28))
 (segment (start 160 101.5) (end 156.5 98) (width 0.2) (layer "F.Cu") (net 28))
 (segment (start 186.921008 102.32) (end 188.071 101.170008) (width 0.2) (layer "F.Cu") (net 25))
 (segment (start 186.895 93.68) (end 191.075 93.68) (width 0.2) (layer "F.Cu") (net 25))
 (segment (start 186.895 102.32) (end 186.921008 102.32) (width 0.2) (layer "F.Cu") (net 25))
 (segment (start 191.075 93.68) (end 191.075 102.32) (width 0.2) (layer "F.Cu") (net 25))
 (segment (start 188.071 101.170008) (end 188.071 94.571) (width 0.2) (layer "F.Cu") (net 25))
 (segment (start 187.18 93.68) (end 186.895 93.68) (width 0.2) (layer "F.Cu") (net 25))
 (segment (start 188.071 94.571) (end 187.18 93.68) (width 0.2) (layer "F.Cu") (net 25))
 (segment (start 162.59 92.8) (end 162.69 92.9) (width 0.2) (layer "F.Cu") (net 4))
 (segment (start 160.45 92.8) (end 162.59 92.8) (width 0.2) (layer "F.Cu") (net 4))
 (segment (start 159.1135 103.3635) (end 160.9245 103.3635) (width 0.2) (layer "F.Cu") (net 10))
 (segment (start 157.5 101.75) (end 159.1135 103.3635) (width 0.2) (layer "F.Cu") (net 10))
 (segment (start 160.9245 103.3635) (end 162.388 101.9) (width 0.2) (layer "F.Cu") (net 10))
 (segment (start 157.5 101.75) (end 149.5 101.75) (width 0.2) (layer "F.Cu") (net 10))
 (segment (start 162.388 101.9) (end 162.69 101.9) (width 0.2) (layer "F.Cu") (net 10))
 (segment (start 184.6375 100.4) (end 184 101.0375) (width 0.2) (layer "F.Cu") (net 20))
 (segment (start 187.5 99.678824) (end 186.778824 100.4) (width 0.2) (layer "F.Cu") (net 20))
 (segment (start 186.32 95.6) (end 186.894999 95.6) (width 0.2) (layer "F.Cu") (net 20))
 (segment (start 186.32 100.4) (end 184.6375 100.4) (width 0.2) (layer "F.Cu") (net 20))
 (segment (start 186.894999 95.6) (end 187.5 96.205001) (width 0.2) (layer "F.Cu") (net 20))
 (segment (start 187.5 96.205001) (end 187.5 99.678824) (width 0.2) (layer "F.Cu") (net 20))
 (segment (start 186.778824 100.4) (end 186.32 100.4) (width 0.2) (layer "F.Cu") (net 20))
 (segment (start 184 103.9625) (end 183 104.9625) (width 0.2) (layer "F.Cu") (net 27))
 (segment (start 183 104.9625) (end 160.5 104.9625) (width 0.2) (layer "F.Cu") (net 27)))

